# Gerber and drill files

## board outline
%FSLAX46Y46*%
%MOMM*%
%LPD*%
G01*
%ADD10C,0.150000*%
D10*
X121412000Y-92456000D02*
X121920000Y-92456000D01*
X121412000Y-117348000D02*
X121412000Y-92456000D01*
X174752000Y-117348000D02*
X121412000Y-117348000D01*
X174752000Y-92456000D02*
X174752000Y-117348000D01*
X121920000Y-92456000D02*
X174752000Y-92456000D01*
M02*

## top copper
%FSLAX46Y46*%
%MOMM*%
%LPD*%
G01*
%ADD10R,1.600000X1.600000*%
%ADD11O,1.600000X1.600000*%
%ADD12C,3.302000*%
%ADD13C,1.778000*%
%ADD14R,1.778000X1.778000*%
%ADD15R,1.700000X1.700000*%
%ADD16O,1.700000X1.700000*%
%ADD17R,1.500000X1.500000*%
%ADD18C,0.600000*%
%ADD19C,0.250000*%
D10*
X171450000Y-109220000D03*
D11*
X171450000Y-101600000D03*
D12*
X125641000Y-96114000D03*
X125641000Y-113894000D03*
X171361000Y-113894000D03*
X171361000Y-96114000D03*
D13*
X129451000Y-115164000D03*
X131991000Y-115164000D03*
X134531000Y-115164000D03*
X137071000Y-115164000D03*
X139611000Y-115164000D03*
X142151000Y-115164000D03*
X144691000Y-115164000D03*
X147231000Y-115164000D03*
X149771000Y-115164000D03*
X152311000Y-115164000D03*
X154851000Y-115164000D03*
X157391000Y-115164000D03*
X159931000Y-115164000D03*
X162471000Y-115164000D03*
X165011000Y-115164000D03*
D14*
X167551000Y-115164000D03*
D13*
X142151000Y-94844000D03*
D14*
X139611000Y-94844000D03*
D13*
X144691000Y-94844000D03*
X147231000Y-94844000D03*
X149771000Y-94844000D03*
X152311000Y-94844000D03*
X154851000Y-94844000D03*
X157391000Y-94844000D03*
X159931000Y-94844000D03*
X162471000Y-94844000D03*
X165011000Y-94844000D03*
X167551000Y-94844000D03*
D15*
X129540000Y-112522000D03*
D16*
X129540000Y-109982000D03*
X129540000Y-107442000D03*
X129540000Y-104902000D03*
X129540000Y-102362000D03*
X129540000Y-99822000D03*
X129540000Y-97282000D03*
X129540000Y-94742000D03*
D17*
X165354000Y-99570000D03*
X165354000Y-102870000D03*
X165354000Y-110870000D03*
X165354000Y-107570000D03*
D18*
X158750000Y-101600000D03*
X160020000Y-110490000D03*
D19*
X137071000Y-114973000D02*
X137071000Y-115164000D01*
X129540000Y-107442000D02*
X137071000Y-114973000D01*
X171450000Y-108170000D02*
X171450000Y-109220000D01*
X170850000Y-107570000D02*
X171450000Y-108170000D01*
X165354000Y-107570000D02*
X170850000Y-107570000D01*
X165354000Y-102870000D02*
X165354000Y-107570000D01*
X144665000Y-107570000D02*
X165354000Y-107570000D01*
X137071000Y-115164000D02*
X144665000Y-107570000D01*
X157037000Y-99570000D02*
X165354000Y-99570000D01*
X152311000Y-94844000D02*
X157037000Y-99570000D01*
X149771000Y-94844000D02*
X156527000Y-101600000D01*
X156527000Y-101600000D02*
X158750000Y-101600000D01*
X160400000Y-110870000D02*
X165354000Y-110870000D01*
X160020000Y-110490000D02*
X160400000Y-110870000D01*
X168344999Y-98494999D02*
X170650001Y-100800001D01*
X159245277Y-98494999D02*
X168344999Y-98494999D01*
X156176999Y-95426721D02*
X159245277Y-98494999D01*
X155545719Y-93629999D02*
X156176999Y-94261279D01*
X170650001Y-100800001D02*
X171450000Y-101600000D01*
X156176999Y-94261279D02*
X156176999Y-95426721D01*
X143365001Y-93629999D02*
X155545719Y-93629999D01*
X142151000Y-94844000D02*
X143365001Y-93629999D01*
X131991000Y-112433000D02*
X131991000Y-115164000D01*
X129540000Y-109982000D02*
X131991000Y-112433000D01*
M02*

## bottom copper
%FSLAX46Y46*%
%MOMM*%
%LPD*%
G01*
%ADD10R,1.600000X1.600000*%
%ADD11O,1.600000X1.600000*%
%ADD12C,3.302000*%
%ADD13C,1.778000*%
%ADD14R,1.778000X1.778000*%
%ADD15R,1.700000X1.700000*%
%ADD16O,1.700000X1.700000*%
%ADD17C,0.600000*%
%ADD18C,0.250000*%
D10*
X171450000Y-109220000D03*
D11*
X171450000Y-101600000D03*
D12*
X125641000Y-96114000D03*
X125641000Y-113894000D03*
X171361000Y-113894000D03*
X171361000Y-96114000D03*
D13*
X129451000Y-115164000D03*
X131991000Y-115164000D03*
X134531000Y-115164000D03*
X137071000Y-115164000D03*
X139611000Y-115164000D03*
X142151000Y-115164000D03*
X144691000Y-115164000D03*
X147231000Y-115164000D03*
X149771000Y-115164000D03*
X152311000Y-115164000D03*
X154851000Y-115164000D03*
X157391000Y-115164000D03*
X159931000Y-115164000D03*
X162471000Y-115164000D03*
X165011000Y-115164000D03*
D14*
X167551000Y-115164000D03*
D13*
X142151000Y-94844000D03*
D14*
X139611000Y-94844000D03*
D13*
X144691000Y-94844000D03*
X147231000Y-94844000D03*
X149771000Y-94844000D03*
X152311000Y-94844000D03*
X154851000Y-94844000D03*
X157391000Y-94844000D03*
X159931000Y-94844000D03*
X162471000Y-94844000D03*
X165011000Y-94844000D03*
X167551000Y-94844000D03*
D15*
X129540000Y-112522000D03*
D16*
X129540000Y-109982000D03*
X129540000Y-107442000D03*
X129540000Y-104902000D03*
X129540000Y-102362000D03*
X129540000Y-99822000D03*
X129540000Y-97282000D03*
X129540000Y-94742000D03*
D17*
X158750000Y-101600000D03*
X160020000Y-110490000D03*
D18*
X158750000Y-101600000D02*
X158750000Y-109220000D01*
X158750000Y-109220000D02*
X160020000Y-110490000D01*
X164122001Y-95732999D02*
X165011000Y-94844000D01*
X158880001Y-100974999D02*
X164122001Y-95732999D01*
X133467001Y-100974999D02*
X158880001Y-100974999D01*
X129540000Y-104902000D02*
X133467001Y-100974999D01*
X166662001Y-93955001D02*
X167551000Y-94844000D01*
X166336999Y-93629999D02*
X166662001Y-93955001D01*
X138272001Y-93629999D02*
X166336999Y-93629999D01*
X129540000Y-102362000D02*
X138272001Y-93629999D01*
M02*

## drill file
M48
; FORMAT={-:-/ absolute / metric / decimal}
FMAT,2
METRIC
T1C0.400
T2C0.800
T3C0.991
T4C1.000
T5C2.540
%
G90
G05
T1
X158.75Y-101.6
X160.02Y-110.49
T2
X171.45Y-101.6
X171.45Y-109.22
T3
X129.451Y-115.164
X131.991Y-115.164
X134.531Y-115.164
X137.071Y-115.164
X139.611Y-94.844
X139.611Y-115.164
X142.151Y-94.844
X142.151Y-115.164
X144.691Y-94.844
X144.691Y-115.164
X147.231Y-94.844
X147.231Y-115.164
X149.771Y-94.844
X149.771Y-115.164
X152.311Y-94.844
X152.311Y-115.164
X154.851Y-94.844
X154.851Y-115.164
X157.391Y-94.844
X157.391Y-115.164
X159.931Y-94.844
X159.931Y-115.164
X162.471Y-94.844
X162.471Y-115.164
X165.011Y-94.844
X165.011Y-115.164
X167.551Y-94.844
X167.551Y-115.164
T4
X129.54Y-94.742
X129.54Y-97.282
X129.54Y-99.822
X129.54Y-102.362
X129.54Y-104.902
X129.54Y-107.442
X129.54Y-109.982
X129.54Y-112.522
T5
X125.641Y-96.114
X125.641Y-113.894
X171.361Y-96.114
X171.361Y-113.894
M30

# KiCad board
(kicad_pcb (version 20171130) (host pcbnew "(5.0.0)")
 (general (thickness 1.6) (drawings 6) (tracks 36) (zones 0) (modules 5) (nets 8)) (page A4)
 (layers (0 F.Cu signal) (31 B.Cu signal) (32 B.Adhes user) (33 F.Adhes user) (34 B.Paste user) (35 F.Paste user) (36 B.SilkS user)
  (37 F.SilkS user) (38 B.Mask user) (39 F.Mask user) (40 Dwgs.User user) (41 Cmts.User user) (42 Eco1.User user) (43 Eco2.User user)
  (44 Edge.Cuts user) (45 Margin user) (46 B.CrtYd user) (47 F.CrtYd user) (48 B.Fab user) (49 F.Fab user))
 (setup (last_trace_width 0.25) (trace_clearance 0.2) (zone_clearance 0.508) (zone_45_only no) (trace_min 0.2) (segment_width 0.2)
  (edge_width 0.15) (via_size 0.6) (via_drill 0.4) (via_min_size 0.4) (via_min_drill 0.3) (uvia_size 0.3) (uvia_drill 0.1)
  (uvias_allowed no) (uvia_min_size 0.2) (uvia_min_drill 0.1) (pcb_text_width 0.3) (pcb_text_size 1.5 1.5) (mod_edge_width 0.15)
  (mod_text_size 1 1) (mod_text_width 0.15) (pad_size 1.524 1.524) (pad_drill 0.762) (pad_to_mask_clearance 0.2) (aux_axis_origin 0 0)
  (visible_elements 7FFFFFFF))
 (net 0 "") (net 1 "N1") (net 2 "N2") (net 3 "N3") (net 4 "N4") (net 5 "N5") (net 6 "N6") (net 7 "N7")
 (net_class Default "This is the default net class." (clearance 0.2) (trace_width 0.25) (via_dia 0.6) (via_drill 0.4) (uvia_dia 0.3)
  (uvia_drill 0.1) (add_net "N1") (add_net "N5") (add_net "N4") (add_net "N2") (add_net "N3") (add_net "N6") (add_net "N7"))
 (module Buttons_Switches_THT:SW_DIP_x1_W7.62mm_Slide (layer F.Cu) (at 171.45 109.22 90)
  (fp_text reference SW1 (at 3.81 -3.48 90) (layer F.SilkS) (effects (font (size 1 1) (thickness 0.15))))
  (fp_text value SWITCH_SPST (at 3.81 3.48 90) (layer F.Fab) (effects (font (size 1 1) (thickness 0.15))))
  (pad 1 thru_hole rect (at 0 0 90) (size 1.6 1.6) (drill 0.8) (layers *.Cu *.Mask) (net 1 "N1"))
  (pad 2 thru_hole oval (at 7.62 0 90) (size 1.6 1.6) (drill 0.8) (layers *.Cu *.Mask) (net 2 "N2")))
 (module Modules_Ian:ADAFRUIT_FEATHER (layer F.Cu) (at 148.501 105.004)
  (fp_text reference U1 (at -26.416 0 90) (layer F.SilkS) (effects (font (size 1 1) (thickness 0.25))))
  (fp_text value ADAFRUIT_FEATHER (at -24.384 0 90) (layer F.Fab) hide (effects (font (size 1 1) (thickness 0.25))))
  (pad "" thru_hole circle (at -22.86 -8.89) (size 3.302 3.302) (drill 2.54) (layers *.Cu *.Mask F.SilkS))
  (pad "" thru_hole circle (at -22.86 8.89) (size 3.302 3.302) (drill 2.54) (layers *.Cu *.Mask F.SilkS))
  (pad "" thru_hole circle (at 22.86 8.89) (size 3.302 3.302) (drill 2.54) (layers *.Cu *.Mask F.SilkS))
  (pad "" thru_hole circle (at 22.86 -8.89) (size 3.302 3.302) (drill 2.54) (layers *.Cu *.Mask F.SilkS))
  (pad 16 thru_hole circle (at -19.05 10.16) (size 1.778 1.778) (drill 0.9906) (layers *.Cu *.Mask F.SilkS))
  (pad 15 thru_hole circle (at -16.51 10.16) (size 1.778 1.778) (drill 0.9906) (layers *.Cu *.Mask F.SilkS) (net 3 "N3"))
  (pad 14 thru_hole circle (at -13.97 10.16) (size 1.778 1.778) (drill 0.9906) (layers *.Cu *.Mask F.SilkS))
  (pad 13 thru_hole circle (at -11.43 10.16) (size 1.778 1.778) (drill 0.9906) (layers *.Cu *.Mask F.SilkS) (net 1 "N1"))
  (pad 12 thru_hole circle (at -8.89 10.16) (size 1.778 1.778) (drill 0.9906) (layers *.Cu *.Mask F.SilkS))
  (pad 11 thru_hole circle (at -6.35 10.16) (size 1.778 1.778) (drill 0.9906) (layers *.Cu *.Mask F.SilkS))
  (pad 10 thru_hole circle (at -3.81 10.16) (size 1.778 1.778) (drill 0.9906) (layers *.Cu *.Mask F.SilkS))
  (pad 9 thru_hole circle (at -1.27 10.16) (size 1.778 1.778) (drill 0.9906) (layers *.Cu *.Mask F.SilkS))
  (pad 8 thru_hole circle (at 1.27 10.16) (size 1.778 1.778) (drill 0.9906) (layers *.Cu *.Mask F.SilkS))
  (pad 7 thru_hole circle (at 3.81 10.16) (size 1.778 1.778) (drill 0.9906) (layers *.Cu *.Mask F.SilkS))
  (pad 6 thru_hole circle (at 6.35 10.16) (size 1.778 1.778) (drill 0.9906) (layers *.Cu *.Mask F.SilkS))
  (pad 5 thru_hole circle (at 8.89 10.16) (size 1.778 1.778) (drill 0.9906) (layers *.Cu *.Mask F.SilkS))
  (pad 4 thru_hole circle (at 11.43 10.16) (size 1.778 1.778) (drill 0.9906) (layers *.Cu *.Mask F.SilkS))
  (pad 3 thru_hole circle (at 13.97 10.16) (size 1.778 1.778) (drill 0.9906) (layers *.Cu *.Mask F.SilkS))
  (pad 2 thru_hole circle (at 16.51 10.16) (size 1.778 1.778) (drill 0.9906) (layers *.Cu *.Mask F.SilkS))
  (pad 1 thru_hole rect (at 19.05 10.16) (size 1.778 1.778) (drill 0.9906) (layers *.Cu *.Mask F.SilkS))
  (pad 18 thru_hole circle (at -6.35 -10.16) (size 1.778 1.778) (drill 0.9906) (layers *.Cu *.Mask F.SilkS) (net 2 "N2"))
  (pad 17 thru_hole rect (at -8.89 -10.16) (size 1.778 1.778) (drill 0.9906) (layers *.Cu *.Mask F.SilkS))
  (pad 19 thru_hole circle (at -3.81 -10.16) (size 1.778 1.778) (drill 0.9906) (layers *.Cu *.Mask F.SilkS))
  (pad 20 thru_hole circle (at -1.27 -10.16) (size 1.778 1.778) (drill 0.9906) (layers *.Cu *.Mask F.SilkS))
  (pad 21 thru_hole circle (at 1.27 -10.16) (size 1.778 1.778) (drill 0.9906) (layers *.Cu *.Mask F.SilkS) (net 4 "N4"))
  (pad 22 thru_hole circle (at 3.81 -10.16) (size 1.778 1.778) (drill 0.9906) (layers *.Cu *.Mask F.SilkS) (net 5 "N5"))
  (pad 23 thru_hole circle (at 6.35 -10.16) (size 1.778 1.778) (drill 0.9906) (layers *.Cu *.Mask F.SilkS))
  (pad 24 thru_hole circle (at 8.89 -10.16) (size 1.778 1.778) (drill 0.9906) (layers *.Cu *.Mask F.SilkS))
  (pad 25 thru_hole circle (at 11.43 -10.16) (size 1.778 1.778) (drill 0.9906) (layers *.Cu *.Mask F.SilkS))
  (pad 26 thru_hole circle (at 13.97 -10.16) (size 1.778 1.778) (drill 0.9906) (layers *.Cu *.Mask F.SilkS))
  (pad 27 thru_hole circle (at 16.51 -10.16) (size 1.778 1.778) (drill 0.9906) (layers *.Cu *.Mask F.SilkS) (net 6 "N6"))
  (pad 28 thru_hole circle (at 19.05 -10.16) (size 1.778 1.778) (drill 0.9906) (layers *.Cu *.Mask F.SilkS) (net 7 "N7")))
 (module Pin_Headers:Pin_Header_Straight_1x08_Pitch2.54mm (layer F.Cu) (at 129.54 112.522 180)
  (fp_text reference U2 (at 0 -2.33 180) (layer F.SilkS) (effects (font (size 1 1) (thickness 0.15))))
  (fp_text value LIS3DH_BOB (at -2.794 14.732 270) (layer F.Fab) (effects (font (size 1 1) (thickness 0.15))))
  (pad 1 thru_hole rect (at 0 0 180) (size 1.7 1.7) (drill 1) (layers *.Cu *.Mask))
  (pad 2 thru_hole oval (at 0 2.54 180) (size 1.7 1.7) (drill 1) (layers *.Cu *.Mask) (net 3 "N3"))
  (pad 3 thru_hole oval (at 0 5.08 180) (size 1.7 1.7) (drill 1) (layers *.Cu *.Mask) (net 1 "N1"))
  (pad 4 thru_hole oval (at 0 7.62 180) (size 1.7 1.7) (drill 1) (layers *.Cu *.Mask) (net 6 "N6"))
  (pad 5 thru_hole oval (at 0 10.16 180) (size 1.7 1.7) (drill 1) (layers *.Cu *.Mask) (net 7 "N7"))
  (pad 6 thru_hole oval (at 0 12.7 180) (size 1.7 1.7) (drill 1) (layers *.Cu *.Mask))
  (pad 7 thru_hole oval (at 0 15.24 180) (size 1.7 1.7) (drill 1) (layers *.Cu *.Mask))
  (pad 8 thru_hole oval (at 0 17.78 180) (size 1.7 1.7) (drill 1) (layers *.Cu *.Mask)))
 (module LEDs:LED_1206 (layer F.Cu) (at 165.354 101.22 90)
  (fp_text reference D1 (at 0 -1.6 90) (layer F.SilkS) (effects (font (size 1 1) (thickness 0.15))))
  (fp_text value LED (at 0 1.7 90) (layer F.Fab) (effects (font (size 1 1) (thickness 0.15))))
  (pad 2 smd rect (at 1.65 0 270) (size 1.5 1.5) (layers F.Cu F.Paste F.Mask) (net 5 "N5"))
  (pad 1 smd rect (at -1.65 0 270) (size 1.5 1.5) (layers F.Cu F.Paste F.Mask) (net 1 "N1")))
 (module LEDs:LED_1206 (layer F.Cu) (at 165.354 109.22 270)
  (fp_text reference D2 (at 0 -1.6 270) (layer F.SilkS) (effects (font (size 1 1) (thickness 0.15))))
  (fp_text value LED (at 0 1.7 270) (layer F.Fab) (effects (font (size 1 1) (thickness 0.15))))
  (pad 2 smd rect (at 1.65 0 90) (size 1.5 1.5) (layers F.Cu F.Paste F.Mask) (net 4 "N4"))
  (pad 1 smd rect (at -1.65 0 90) (size 1.5 1.5) (layers F.Cu F.Paste F.Mask) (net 1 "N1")))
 (gr_line (start 121.412 92.456) (end 121.92 92.456) (angle 90) (layer Edge.Cuts) (width 0.15))
 (gr_line (start 121.412 117.348) (end 121.412 92.456) (angle 90) (layer Edge.Cuts) (width 0.15))
 (gr_line (start 174.752 117.348) (end 121.412 117.348) (angle 90) (layer Edge.Cuts) (width 0.15))
 (gr_line (start 174.752 92.456) (end 174.752 117.348) (angle 90) (layer Edge.Cuts) (width 0.15))
 (gr_line (start 121.92 92.456) (end 174.752 92.456) (angle 90) (layer Edge.Cuts) (width 0.15))
 (segment (start 137.071 114.973) (end 137.071 115.164) (width 0.25) (layer F.Cu) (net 1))
 (segment (start 129.54 107.442) (end 137.071 114.973) (width 0.25) (layer F.Cu) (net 1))
 (segment (start 171.45 108.17) (end 171.45 109.22) (width 0.25) (layer F.Cu) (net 1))
 (segment (start 170.85 107.57) (end 171.45 108.17) (width 0.25) (layer F.Cu) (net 1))
 (segment (start 165.354 107.57) (end 170.85 107.57) (width 0.25) (layer F.Cu) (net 1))
 (segment (start 165.354 102.87) (end 165.354 107.57) (width 0.25) (layer F.Cu) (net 1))
 (segment (start 144.665 107.57) (end 165.354 107.57) (width 0.25) (layer F.Cu) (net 1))
 (segment (start 137.071 115.164) (end 144.665 107.57) (width 0.25) (layer F.Cu) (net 1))
 (segment (start 157.037 99.57) (end 165.354 99.57) (width 0.25) (layer F.Cu) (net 5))
 (segment (start 152.311 94.844) (end 157.037 99.57) (width 0.25) (layer F.Cu) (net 5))
 (via (at 158.75 101.6) (size 0.6) (drill 0.4) (layers F.Cu B.Cu) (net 4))
 (segment (start 149.771 94.844) (end 156.527 101.6) (width 0.25) (layer F.Cu) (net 4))
 (segment (start 156.527 101.6) (end 158.75 101.6) (width 0.25) (layer F.Cu) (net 4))
 (via (at 160.02 110.49) (size 0.6) (drill 0.4) (layers F.Cu B.Cu) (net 4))
 (segment (start 158.75 101.6) (end 158.75 109.22) (width 0.25) (layer B.Cu) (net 4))
 (segment (start 158.75 109.22) (end 160.02 110.49) (width 0.25) (layer B.Cu) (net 4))
 (segment (start 160.4 110.87) (end 165.354 110.87) (width 0.25) (layer F.Cu) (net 4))
 (segment (start 160.02 110.49) (end 160.4 110.87) (width 0.25) (layer F.Cu) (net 4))
 (segment (start 168.344999 98.494999) (end 170.650001 100.800001) (width 0.25) (layer F.Cu) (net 2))
 (segment (start 159.245277 98.494999) (end 168.344999 98.494999) (width 0.25) (layer F.Cu) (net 2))
 (segment (start 156.176999 95.426721) (end 159.245277 98.494999) (width 0.25) (layer F.Cu) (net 2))
 (segment (start 155.545719 93.629999) (end 156.176999 94.261279) (width 0.25) (layer F.Cu) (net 2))
 (segment (start 170.650001 100.800001) (end 171.45 101.6) (width 0.25) (layer F.Cu) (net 2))
 (segment (start 156.176999 94.261279) (end 156.176999 95.426721) (width 0.25) (layer F.Cu) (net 2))
 (segment (start 143.365001 93.629999) (end 155.545719 93.629999) (width 0.25) (layer F.Cu) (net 2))
 (segment (start 142.151 94.844) (end 143.365001 93.629999) (width 0.25) (layer F.Cu) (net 2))
 (segment (start 131.991 112.433) (end 131.991 115.164) (width 0.25) (layer F.Cu) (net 3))
 (segment (start 129.54 109.982) (end 131.991 112.433) (width 0.25) (layer F.Cu) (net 3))
 (segment (start 164.122001 95.732999) (end 165.011 94.844) (width 0.25) (layer B.Cu) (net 6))
 (segment (start 158.880001 100.974999) (end 164.122001 95.732999) (width 0.25) (layer B.Cu) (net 6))
 (segment (start 133.467001 100.974999) (end 158.880001 100.974999) (width 0.25) (layer B.Cu) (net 6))
 (segment (start 129.54 104.902) (end 133.467001 100.974999) (width 0.25) (layer B.Cu) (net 6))
 (segment (start 166.662001 93.955001) (end 167.551 94.844) (width 0.25) (layer B.Cu) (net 7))
 (segment (start 166.336999 93.629999) (end 166.662001 93.955001) (width 0.25) (layer B.Cu) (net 7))
 (segment (start 138.272001 93.629999) (end 166.336999 93.629999) (width 0.25) (layer B.Cu) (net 7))
 (segment (start 129.54 102.362) (end 138.272001 93.629999) (width 0.25) (layer B.Cu) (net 7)))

